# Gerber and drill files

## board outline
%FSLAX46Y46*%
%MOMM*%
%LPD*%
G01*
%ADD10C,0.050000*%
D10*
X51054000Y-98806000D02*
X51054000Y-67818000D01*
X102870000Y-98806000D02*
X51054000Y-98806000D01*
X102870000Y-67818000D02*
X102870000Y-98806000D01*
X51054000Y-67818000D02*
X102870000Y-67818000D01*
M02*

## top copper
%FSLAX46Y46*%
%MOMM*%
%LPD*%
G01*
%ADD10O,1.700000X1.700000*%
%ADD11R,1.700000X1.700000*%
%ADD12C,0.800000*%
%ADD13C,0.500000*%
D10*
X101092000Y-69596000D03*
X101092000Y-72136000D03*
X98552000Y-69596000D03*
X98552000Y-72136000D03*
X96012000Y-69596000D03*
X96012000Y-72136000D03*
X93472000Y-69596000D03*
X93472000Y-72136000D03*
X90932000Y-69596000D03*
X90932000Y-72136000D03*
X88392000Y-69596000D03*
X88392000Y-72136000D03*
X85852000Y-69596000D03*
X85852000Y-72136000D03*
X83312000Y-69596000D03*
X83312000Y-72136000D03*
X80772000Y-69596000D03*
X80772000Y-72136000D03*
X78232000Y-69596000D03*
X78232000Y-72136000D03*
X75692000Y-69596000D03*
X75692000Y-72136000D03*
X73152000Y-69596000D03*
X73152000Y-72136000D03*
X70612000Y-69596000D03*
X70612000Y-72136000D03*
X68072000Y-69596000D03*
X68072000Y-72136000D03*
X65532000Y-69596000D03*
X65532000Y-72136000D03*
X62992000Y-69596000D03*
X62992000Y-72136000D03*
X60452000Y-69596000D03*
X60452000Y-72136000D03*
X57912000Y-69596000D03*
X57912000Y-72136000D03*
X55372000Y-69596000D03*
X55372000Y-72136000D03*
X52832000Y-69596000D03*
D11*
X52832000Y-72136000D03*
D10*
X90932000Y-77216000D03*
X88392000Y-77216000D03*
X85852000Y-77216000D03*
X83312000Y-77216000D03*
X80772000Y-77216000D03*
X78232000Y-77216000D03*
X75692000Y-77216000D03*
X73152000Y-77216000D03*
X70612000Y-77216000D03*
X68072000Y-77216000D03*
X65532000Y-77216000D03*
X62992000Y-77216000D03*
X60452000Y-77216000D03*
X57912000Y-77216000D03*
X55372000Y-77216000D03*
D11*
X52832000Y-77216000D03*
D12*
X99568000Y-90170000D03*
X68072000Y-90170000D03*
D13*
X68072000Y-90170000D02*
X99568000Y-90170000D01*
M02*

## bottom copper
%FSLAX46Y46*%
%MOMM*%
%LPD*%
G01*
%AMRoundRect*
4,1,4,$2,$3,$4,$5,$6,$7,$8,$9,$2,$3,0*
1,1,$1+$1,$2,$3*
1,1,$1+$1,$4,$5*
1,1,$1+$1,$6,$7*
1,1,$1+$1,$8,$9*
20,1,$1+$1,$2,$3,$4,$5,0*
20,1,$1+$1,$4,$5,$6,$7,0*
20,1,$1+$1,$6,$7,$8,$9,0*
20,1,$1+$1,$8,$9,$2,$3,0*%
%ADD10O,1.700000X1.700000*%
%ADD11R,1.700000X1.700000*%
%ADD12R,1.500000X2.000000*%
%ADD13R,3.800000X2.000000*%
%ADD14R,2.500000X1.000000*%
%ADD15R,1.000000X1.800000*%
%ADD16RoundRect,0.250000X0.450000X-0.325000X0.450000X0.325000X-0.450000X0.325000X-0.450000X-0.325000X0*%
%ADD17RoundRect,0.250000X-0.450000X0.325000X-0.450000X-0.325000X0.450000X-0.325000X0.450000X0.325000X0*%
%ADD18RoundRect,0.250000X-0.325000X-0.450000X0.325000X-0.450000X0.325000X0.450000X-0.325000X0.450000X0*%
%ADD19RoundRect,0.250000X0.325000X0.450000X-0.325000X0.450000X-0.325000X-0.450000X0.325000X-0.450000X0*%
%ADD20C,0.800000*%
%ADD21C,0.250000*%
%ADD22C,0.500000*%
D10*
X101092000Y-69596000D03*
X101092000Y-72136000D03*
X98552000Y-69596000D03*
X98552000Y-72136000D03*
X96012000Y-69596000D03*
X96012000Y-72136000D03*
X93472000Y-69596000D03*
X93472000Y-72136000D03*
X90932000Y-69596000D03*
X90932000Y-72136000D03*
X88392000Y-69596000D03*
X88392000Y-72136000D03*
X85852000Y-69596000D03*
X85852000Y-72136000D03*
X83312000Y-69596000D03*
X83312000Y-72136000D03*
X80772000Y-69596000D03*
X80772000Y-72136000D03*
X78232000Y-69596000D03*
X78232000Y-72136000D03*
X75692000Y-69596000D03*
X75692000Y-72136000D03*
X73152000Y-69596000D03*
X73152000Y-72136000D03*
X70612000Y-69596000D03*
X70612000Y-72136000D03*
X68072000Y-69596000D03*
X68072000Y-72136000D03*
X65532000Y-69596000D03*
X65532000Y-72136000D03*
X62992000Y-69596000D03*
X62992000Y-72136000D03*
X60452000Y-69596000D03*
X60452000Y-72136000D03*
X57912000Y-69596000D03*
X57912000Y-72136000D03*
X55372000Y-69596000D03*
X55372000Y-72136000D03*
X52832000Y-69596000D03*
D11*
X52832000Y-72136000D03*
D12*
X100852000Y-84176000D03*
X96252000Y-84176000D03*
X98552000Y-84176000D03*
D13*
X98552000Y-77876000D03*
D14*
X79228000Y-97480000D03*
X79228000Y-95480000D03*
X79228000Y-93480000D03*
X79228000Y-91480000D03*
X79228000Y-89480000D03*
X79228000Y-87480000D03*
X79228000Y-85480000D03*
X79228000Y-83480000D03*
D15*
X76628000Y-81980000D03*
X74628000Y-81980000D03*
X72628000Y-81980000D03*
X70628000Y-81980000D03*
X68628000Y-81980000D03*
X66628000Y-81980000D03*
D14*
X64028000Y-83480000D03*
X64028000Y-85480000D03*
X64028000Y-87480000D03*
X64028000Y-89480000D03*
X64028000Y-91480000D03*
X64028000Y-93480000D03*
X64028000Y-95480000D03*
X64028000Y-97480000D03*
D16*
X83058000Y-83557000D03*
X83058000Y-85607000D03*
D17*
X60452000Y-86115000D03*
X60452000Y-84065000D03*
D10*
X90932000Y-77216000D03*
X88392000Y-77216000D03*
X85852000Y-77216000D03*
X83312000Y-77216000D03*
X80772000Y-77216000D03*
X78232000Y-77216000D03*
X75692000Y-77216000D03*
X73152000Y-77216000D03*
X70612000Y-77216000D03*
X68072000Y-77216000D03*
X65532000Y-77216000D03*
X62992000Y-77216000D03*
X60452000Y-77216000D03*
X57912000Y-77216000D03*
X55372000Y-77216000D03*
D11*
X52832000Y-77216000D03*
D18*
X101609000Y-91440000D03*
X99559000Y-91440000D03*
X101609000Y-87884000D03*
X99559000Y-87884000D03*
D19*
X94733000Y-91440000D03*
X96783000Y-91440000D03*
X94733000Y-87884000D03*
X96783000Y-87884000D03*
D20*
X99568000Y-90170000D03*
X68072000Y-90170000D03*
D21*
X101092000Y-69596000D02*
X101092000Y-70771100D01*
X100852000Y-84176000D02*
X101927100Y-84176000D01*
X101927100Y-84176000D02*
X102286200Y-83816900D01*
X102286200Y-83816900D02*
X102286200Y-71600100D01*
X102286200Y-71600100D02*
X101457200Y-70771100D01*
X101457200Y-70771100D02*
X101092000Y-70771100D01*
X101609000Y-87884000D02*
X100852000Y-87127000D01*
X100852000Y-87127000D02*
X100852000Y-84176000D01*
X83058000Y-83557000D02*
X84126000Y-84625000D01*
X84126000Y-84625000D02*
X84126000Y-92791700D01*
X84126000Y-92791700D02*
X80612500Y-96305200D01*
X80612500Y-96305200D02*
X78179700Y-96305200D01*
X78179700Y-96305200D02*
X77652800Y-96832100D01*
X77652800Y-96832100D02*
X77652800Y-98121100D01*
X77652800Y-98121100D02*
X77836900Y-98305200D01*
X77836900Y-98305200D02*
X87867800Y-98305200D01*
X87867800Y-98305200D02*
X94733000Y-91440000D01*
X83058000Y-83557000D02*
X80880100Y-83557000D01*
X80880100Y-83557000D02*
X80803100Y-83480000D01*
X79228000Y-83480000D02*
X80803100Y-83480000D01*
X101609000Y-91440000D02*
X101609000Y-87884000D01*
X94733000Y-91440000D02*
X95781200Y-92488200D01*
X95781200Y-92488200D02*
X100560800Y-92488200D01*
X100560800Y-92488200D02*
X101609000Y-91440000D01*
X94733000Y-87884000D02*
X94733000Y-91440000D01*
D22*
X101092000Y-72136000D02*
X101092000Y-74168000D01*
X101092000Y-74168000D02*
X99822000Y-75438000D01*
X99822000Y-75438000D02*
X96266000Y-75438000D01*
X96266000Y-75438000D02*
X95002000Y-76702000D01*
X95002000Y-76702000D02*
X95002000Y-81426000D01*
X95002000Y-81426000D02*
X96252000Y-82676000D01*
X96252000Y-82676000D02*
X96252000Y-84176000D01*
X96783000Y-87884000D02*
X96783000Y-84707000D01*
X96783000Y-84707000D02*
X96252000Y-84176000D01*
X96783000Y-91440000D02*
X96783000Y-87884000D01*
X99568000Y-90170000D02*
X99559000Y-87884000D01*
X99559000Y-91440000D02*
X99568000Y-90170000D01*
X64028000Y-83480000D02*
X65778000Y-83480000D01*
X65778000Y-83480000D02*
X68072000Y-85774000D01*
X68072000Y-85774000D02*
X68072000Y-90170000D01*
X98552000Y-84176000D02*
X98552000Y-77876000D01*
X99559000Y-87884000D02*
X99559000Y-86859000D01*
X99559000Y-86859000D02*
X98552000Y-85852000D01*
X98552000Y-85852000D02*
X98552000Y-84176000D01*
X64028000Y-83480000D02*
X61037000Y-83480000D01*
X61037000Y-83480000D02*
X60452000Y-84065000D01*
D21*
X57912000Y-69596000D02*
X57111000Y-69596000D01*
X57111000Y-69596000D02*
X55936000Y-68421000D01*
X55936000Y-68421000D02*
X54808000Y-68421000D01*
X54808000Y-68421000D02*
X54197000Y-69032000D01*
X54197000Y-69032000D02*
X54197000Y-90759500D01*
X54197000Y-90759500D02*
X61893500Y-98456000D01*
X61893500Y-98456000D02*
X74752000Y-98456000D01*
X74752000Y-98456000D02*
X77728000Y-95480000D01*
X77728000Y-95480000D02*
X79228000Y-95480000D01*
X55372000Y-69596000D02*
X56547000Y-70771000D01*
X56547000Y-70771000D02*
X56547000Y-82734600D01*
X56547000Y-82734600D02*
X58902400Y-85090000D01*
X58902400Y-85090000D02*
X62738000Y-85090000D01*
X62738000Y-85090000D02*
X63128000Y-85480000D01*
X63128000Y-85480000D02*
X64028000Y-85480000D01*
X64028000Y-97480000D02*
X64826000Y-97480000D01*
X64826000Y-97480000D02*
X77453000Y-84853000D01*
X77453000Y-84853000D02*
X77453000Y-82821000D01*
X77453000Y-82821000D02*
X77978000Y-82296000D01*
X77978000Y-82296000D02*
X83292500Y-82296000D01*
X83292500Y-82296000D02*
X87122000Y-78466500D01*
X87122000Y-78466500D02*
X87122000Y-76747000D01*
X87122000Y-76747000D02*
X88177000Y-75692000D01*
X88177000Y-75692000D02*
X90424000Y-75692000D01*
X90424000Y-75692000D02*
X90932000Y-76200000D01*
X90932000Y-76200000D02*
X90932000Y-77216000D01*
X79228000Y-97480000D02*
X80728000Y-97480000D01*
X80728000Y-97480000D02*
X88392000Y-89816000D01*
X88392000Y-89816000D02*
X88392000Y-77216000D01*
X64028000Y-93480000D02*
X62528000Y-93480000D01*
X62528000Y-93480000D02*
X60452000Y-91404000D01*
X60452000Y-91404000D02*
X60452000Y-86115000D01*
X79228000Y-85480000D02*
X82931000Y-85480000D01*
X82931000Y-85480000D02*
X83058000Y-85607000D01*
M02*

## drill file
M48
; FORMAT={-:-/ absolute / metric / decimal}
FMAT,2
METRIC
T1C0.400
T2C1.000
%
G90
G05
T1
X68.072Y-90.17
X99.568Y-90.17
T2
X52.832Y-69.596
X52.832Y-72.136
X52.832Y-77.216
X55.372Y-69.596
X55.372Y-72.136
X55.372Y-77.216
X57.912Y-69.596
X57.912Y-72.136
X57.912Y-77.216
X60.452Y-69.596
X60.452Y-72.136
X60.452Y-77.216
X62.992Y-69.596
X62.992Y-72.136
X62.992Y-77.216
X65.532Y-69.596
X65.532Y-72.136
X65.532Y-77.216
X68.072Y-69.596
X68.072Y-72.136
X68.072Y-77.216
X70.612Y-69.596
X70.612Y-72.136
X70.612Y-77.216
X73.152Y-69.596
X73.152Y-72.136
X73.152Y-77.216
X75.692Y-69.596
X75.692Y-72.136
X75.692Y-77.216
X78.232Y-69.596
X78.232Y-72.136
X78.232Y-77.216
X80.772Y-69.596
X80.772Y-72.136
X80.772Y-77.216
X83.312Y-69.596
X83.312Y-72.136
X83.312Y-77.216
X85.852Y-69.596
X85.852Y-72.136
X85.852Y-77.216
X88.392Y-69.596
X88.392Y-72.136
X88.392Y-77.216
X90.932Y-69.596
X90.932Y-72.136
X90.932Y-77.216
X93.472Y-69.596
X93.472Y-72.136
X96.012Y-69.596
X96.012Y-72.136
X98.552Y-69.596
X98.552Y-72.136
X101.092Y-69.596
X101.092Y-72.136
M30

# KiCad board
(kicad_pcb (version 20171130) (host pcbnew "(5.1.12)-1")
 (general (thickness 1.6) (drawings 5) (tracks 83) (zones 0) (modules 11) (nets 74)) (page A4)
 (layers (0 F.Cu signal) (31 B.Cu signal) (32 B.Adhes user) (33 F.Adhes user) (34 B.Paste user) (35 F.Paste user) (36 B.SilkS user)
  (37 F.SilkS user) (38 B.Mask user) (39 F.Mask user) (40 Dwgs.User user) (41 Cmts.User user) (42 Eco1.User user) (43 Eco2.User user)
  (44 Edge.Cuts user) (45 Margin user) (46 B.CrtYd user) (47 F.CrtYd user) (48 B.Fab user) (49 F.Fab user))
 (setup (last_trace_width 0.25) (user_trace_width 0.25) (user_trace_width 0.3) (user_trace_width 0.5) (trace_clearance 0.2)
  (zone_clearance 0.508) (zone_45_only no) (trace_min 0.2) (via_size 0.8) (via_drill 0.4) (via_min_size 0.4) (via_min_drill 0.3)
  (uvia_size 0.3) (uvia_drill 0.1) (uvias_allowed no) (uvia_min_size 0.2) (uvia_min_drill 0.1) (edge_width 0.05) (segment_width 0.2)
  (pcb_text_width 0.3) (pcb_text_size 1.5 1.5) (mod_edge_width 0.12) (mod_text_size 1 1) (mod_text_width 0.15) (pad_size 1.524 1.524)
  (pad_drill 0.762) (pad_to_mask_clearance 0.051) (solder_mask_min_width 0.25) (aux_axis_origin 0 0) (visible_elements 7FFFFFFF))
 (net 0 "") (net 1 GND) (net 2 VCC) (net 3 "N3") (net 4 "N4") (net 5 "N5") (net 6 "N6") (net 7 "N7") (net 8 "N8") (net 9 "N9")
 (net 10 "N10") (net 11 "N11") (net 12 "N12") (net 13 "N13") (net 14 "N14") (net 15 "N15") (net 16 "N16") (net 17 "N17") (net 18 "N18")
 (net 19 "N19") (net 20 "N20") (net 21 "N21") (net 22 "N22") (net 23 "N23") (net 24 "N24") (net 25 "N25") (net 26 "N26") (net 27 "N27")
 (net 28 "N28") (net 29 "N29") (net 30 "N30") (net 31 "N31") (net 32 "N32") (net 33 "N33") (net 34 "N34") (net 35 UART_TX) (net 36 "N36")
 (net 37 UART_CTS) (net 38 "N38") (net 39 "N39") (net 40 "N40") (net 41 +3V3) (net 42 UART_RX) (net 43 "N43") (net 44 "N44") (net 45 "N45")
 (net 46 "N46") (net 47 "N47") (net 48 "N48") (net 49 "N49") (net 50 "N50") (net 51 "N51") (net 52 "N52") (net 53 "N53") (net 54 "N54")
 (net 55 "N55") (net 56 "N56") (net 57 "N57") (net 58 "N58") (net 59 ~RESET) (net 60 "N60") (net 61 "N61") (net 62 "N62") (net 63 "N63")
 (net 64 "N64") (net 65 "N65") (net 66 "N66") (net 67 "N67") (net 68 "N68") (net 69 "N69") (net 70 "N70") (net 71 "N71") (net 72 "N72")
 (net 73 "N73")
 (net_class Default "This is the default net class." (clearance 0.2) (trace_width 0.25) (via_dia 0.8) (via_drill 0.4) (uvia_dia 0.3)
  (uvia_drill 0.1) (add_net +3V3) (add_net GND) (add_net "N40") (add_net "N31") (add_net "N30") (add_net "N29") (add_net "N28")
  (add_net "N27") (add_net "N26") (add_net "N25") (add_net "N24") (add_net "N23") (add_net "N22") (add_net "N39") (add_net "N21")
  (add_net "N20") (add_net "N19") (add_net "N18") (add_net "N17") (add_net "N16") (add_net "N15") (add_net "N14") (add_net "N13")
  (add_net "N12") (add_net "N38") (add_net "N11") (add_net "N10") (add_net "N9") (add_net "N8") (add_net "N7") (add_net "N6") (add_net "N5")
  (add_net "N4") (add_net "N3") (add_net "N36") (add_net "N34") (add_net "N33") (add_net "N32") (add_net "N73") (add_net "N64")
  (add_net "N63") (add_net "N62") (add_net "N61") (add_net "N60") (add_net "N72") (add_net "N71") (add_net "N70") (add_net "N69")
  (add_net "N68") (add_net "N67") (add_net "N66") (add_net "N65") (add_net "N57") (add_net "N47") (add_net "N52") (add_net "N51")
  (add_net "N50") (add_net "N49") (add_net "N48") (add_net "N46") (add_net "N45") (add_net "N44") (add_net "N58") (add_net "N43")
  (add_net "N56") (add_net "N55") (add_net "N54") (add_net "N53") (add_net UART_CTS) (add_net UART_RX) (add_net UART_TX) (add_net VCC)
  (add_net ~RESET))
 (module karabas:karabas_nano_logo (layer F.Cu) (at 83.566 92.456)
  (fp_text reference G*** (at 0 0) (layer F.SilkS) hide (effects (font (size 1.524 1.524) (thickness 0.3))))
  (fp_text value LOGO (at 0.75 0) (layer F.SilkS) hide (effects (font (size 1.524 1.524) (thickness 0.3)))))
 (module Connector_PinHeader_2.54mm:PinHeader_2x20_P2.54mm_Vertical (layer F.Cu) (at 52.832 72.136 90)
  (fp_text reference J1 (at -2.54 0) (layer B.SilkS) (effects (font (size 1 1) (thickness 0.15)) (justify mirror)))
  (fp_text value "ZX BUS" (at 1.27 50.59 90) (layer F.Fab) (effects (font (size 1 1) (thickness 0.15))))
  (pad 40 thru_hole oval (at 2.54 48.26 90) (size 1.7 1.7) (drill 1) (layers *.Cu *.Mask) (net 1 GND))
  (pad 39 thru_hole oval (at 0 48.26 90) (size 1.7 1.7) (drill 1) (layers *.Cu *.Mask) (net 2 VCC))
  (pad 38 thru_hole oval (at 2.54 45.72 90) (size 1.7 1.7) (drill 1) (layers *.Cu *.Mask) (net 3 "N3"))
  (pad 37 thru_hole oval (at 0 45.72 90) (size 1.7 1.7) (drill 1) (layers *.Cu *.Mask) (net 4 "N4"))
  (pad 36 thru_hole oval (at 2.54 43.18 90) (size 1.7 1.7) (drill 1) (layers *.Cu *.Mask) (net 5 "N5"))
  (pad 35 thru_hole oval (at 0 43.18 90) (size 1.7 1.7) (drill 1) (layers *.Cu *.Mask) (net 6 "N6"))
  (pad 34 thru_hole oval (at 2.54 40.64 90) (size 1.7 1.7) (drill 1) (layers *.Cu *.Mask) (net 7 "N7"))
  (pad 33 thru_hole oval (at 0 40.64 90) (size 1.7 1.7) (drill 1) (layers *.Cu *.Mask) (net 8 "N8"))
  (pad 32 thru_hole oval (at 2.54 38.1 90) (size 1.7 1.7) (drill 1) (layers *.Cu *.Mask) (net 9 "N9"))
  (pad 31 thru_hole oval (at 0 38.1 90) (size 1.7 1.7) (drill 1) (layers *.Cu *.Mask) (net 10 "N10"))
  (pad 30 thru_hole oval (at 2.54 35.56 90) (size 1.7 1.7) (drill 1) (layers *.Cu *.Mask) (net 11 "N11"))
  (pad 29 thru_hole oval (at 0 35.56 90) (size 1.7 1.7) (drill 1) (layers *.Cu *.Mask) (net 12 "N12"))
  (pad 28 thru_hole oval (at 2.54 33.02 90) (size 1.7 1.7) (drill 1) (layers *.Cu *.Mask) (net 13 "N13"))
  (pad 27 thru_hole oval (at 0 33.02 90) (size 1.7 1.7) (drill 1) (layers *.Cu *.Mask) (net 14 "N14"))
  (pad 26 thru_hole oval (at 2.54 30.48 90) (size 1.7 1.7) (drill 1) (layers *.Cu *.Mask) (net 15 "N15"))
  (pad 25 thru_hole oval (at 0 30.48 90) (size 1.7 1.7) (drill 1) (layers *.Cu *.Mask) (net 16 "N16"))
  (pad 24 thru_hole oval (at 2.54 27.94 90) (size 1.7 1.7) (drill 1) (layers *.Cu *.Mask) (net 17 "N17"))
  (pad 23 thru_hole oval (at 0 27.94 90) (size 1.7 1.7) (drill 1) (layers *.Cu *.Mask) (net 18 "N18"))
  (pad 22 thru_hole oval (at 2.54 25.4 90) (size 1.7 1.7) (drill 1) (layers *.Cu *.Mask) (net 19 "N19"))
  (pad 21 thru_hole oval (at 0 25.4 90) (size 1.7 1.7) (drill 1) (layers *.Cu *.Mask) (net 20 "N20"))
  (pad 20 thru_hole oval (at 2.54 22.86 90) (size 1.7 1.7) (drill 1) (layers *.Cu *.Mask) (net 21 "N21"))
  (pad 19 thru_hole oval (at 0 22.86 90) (size 1.7 1.7) (drill 1) (layers *.Cu *.Mask) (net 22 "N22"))
  (pad 18 thru_hole oval (at 2.54 20.32 90) (size 1.7 1.7) (drill 1) (layers *.Cu *.Mask) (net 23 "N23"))
  (pad 17 thru_hole oval (at 0 20.32 90) (size 1.7 1.7) (drill 1) (layers *.Cu *.Mask) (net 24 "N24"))
  (pad 16 thru_hole oval (at 2.54 17.78 90) (size 1.7 1.7) (drill 1) (layers *.Cu *.Mask) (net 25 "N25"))
  (pad 15 thru_hole oval (at 0 17.78 90) (size 1.7 1.7) (drill 1) (layers *.Cu *.Mask) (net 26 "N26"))
  (pad 14 thru_hole oval (at 2.54 15.24 90) (size 1.7 1.7) (drill 1) (layers *.Cu *.Mask) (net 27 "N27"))
  (pad 13 thru_hole oval (at 0 15.24 90) (size 1.7 1.7) (drill 1) (layers *.Cu *.Mask) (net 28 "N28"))
  (pad 12 thru_hole oval (at 2.54 12.7 90) (size 1.7 1.7) (drill 1) (layers *.Cu *.Mask) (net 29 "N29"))
  (pad 11 thru_hole oval (at 0 12.7 90) (size 1.7 1.7) (drill 1) (layers *.Cu *.Mask) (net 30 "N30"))
  (pad 10 thru_hole oval (at 2.54 10.16 90) (size 1.7 1.7) (drill 1) (layers *.Cu *.Mask) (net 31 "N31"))
  (pad 9 thru_hole oval (at 0 10.16 90) (size 1.7 1.7) (drill 1) (layers *.Cu *.Mask) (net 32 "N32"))
  (pad 8 thru_hole oval (at 2.54 7.62 90) (size 1.7 1.7) (drill 1) (layers *.Cu *.Mask) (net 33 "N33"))
  (pad 7 thru_hole oval (at 0 7.62 90) (size 1.7 1.7) (drill 1) (layers *.Cu *.Mask) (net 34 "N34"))
  (pad 6 thru_hole oval (at 2.54 5.08 90) (size 1.7 1.7) (drill 1) (layers *.Cu *.Mask) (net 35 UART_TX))
  (pad 5 thru_hole oval (at 0 5.08 90) (size 1.7 1.7) (drill 1) (layers *.Cu *.Mask) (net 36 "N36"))
  (pad 4 thru_hole oval (at 2.54 2.54 90) (size 1.7 1.7) (drill 1) (layers *.Cu *.Mask) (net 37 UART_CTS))
  (pad 3 thru_hole oval (at 0 2.54 90) (size 1.7 1.7) (drill 1) (layers *.Cu *.Mask) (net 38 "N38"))
  (pad 2 thru_hole oval (at 2.54 0 90) (size 1.7 1.7) (drill 1) (layers *.Cu *.Mask) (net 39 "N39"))
  (pad 1 thru_hole rect (at 0 0 90) (size 1.7 1.7) (drill 1) (layers *.Cu *.Mask) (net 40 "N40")))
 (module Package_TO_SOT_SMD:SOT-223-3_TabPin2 (layer B.Cu) (at 98.552 81.026 90)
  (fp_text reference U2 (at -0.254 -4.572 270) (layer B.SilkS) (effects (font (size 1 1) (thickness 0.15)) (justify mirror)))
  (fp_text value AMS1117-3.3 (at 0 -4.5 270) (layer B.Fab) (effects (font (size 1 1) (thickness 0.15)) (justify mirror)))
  (pad 1 smd rect (at -3.15 2.3 90) (size 2 1.5) (layers B.Cu B.Paste B.Mask) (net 1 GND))
  (pad 3 smd rect (at -3.15 -2.3 90) (size 2 1.5) (layers B.Cu B.Paste B.Mask) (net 2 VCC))
  (pad 2 smd rect (at -3.15 0 90) (size 2 1.5) (layers B.Cu B.Paste B.Mask) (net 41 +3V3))
  (pad 2 smd rect (at 3.15 0 90) (size 2 3.8) (layers B.Cu B.Paste B.Mask) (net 41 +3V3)))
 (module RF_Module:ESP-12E (layer B.Cu) (at 71.628 93.98)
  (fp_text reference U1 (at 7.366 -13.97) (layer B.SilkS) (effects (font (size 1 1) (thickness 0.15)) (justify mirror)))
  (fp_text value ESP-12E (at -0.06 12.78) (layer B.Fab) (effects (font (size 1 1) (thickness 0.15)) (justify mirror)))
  (pad 22 smd rect (at 7.6 3.5) (size 2.5 1) (layers B.Cu B.Paste B.Mask) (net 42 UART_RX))
  (pad 21 smd rect (at 7.6 1.5) (size 2.5 1) (layers B.Cu B.Paste B.Mask) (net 35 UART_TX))
  (pad 20 smd rect (at 7.6 -0.5) (size 2.5 1) (layers B.Cu B.Paste B.Mask) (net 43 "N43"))
  (pad 19 smd rect (at 7.6 -2.5) (size 2.5 1) (layers B.Cu B.Paste B.Mask) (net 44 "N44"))
  (pad 18 smd rect (at 7.6 -4.5) (size 2.5 1) (layers B.Cu B.Paste B.Mask) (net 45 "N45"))
  (pad 17 smd rect (at 7.6 -6.5) (size 2.5 1) (layers B.Cu B.Paste B.Mask) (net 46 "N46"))
  (pad 16 smd rect (at 7.6 -8.5) (size 2.5 1) (layers B.Cu B.Paste B.Mask) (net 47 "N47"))
  (pad 15 smd rect (at 7.6 -10.5) (size 2.5 1) (layers B.Cu B.Paste B.Mask) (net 1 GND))
  (pad 14 smd rect (at 5 -12) (size 1 1.8) (layers B.Cu B.Paste B.Mask) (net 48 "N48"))
  (pad 13 smd rect (at 3 -12) (size 1 1.8) (layers B.Cu B.Paste B.Mask) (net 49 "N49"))
  (pad 12 smd rect (at 1 -12) (size 1 1.8) (layers B.Cu B.Paste B.Mask) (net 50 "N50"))
  (pad 11 smd rect (at -1 -12) (size 1 1.8) (layers B.Cu B.Paste B.Mask) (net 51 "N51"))
  (pad 10 smd rect (at -3 -12) (size 1 1.8) (layers B.Cu B.Paste B.Mask) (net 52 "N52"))
  (pad 9 smd rect (at -5 -12) (size 1 1.8) (layers B.Cu B.Paste B.Mask) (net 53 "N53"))
  (pad 8 smd rect (at -7.6 -10.5) (size 2.5 1) (layers B.Cu B.Paste B.Mask) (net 41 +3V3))
  (pad 7 smd rect (at -7.6 -8.5) (size 2.5 1) (layers B.Cu B.Paste B.Mask) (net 37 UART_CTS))
  (pad 6 smd rect (at -7.6 -6.5) (size 2.5 1) (layers B.Cu B.Paste B.Mask) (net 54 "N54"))
  (pad 5 smd rect (at -7.6 -4.5) (size 2.5 1) (layers B.Cu B.Paste B.Mask) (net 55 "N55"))
  (pad 4 smd rect (at -7.6 -2.5) (size 2.5 1) (layers B.Cu B.Paste B.Mask) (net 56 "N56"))
  (pad 3 smd rect (at -7.6 -0.5) (size 2.5 1) (layers B.Cu B.Paste B.Mask) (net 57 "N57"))
  (pad 2 smd rect (at -7.6 1.5) (size 2.5 1) (layers B.Cu B.Paste B.Mask) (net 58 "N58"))
  (pad 1 smd rect (at -7.6 3.5) (size 2.5 1) (layers B.Cu B.Paste B.Mask) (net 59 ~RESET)))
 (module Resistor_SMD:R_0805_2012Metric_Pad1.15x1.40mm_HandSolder (layer B.Cu) (at 83.058 84.582 90)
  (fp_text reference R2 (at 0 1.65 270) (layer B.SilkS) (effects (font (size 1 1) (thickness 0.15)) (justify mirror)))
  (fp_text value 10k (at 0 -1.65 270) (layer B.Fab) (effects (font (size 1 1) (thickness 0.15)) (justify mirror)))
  (pad 2 smd roundrect (at 1.025 0 90) (size 1.15 1.4) (layers B.Cu B.Paste B.Mask) (roundrect_rratio 0.217391) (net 1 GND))
  (pad 1 smd roundrect (at -1.025 0 90) (size 1.15 1.4) (layers B.Cu B.Paste B.Mask) (roundrect_rratio 0.217391) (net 47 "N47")))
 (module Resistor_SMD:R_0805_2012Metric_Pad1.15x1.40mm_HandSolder (layer B.Cu) (at 60.452 85.09 270)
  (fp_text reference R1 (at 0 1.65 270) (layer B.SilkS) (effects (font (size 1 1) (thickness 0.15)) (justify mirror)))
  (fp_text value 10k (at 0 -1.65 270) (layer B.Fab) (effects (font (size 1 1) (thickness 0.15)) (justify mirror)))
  (pad 2 smd roundrect (at 1.025 0 270) (size 1.15 1.4) (layers B.Cu B.Paste B.Mask) (roundrect_rratio 0.217391) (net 57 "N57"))
  (pad 1 smd roundrect (at -1.025 0 270) (size 1.15 1.4) (layers B.Cu B.Paste B.Mask) (roundrect_rratio 0.217391) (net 41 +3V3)))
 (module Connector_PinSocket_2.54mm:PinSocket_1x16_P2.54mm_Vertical (layer F.Cu) (at 52.832 77.216 90)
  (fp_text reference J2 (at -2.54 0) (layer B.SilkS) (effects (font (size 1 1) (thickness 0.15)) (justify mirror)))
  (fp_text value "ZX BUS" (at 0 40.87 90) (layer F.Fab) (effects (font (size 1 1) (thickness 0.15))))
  (pad 16 thru_hole oval (at 0 38.1 90) (size 1.7 1.7) (drill 1) (layers *.Cu *.Mask) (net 59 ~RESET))
  (pad 15 thru_hole oval (at 0 35.56 90) (size 1.7 1.7) (drill 1) (layers *.Cu *.Mask) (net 42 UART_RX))
  (pad 14 thru_hole oval (at 0 33.02 90) (size 1.7 1.7) (drill 1) (layers *.Cu *.Mask) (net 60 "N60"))
  (pad 13 thru_hole oval (at 0 30.48 90) (size 1.7 1.7) (drill 1) (layers *.Cu *.Mask) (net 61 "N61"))
  (pad 12 thru_hole oval (at 0 27.94 90) (size 1.7 1.7) (drill 1) (layers *.Cu *.Mask) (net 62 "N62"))
  (pad 11 thru_hole oval (at 0 25.4 90) (size 1.7 1.7) (drill 1) (layers *.Cu *.Mask) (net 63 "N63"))
  (pad 10 thru_hole oval (at 0 22.86 90) (size 1.7 1.7) (drill 1) (layers *.Cu *.Mask) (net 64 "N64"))
  (pad 9 thru_hole oval (at 0 20.32 90) (size 1.7 1.7) (drill 1) (layers *.Cu *.Mask) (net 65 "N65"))
  (pad 8 thru_hole oval (at 0 17.78 90) (size 1.7 1.7) (drill 1) (layers *.Cu *.Mask) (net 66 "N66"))
  (pad 7 thru_hole oval (at 0 15.24 90) (size 1.7 1.7) (drill 1) (layers *.Cu *.Mask) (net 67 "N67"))
  (pad 6 thru_hole oval (at 0 12.7 90) (size 1.7 1.7) (drill 1) (layers *.Cu *.Mask) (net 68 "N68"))
  (pad 5 thru_hole oval (at 0 10.16 90) (size 1.7 1.7) (drill 1) (layers *.Cu *.Mask) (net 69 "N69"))
  (pad 4 thru_hole oval (at 0 7.62 90) (size 1.7 1.7) (drill 1) (layers *.Cu *.Mask) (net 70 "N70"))
  (pad 3 thru_hole oval (at 0 5.08 90) (size 1.7 1.7) (drill 1) (layers *.Cu *.Mask) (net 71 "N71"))
  (pad 2 thru_hole oval (at 0 2.54 90) (size 1.7 1.7) (drill 1) (layers *.Cu *.Mask) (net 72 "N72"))
  (pad 1 thru_hole rect (at 0 0 90) (size 1.7 1.7) (drill 1) (layers *.Cu *.Mask) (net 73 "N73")))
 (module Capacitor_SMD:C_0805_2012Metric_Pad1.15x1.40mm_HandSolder (layer B.Cu) (at 100.584 91.44)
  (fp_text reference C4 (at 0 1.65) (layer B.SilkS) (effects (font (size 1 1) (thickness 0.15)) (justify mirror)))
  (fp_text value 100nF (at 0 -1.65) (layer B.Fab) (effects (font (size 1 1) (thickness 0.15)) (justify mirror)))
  (pad 2 smd roundrect (at 1.025 0) (size 1.15 1.4) (layers B.Cu B.Paste B.Mask) (roundrect_rratio 0.217391) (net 1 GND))
  (pad 1 smd roundrect (at -1.025 0) (size 1.15 1.4) (layers B.Cu B.Paste B.Mask) (roundrect_rratio 0.217391) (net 41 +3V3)))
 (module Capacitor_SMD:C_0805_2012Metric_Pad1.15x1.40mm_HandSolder (layer B.Cu) (at 100.584 87.884)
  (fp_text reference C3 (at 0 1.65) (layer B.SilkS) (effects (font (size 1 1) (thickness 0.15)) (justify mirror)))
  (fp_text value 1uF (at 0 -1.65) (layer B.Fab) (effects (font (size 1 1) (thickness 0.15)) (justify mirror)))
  (pad 2 smd roundrect (at 1.025 0) (size 1.15 1.4) (layers B.Cu B.Paste B.Mask) (roundrect_rratio 0.217391) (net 1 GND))
  (pad 1 smd roundrect (at -1.025 0) (size 1.15 1.4) (layers B.Cu B.Paste B.Mask) (roundrect_rratio 0.217391) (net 41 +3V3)))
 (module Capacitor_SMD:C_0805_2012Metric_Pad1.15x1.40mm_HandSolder (layer B.Cu) (at 95.758 91.44 180)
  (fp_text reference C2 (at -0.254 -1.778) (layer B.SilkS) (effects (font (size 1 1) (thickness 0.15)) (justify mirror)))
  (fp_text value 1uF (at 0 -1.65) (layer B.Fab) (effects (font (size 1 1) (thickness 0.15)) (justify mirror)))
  (pad 2 smd roundrect (at 1.025 0 180) (size 1.15 1.4) (layers B.Cu B.Paste B.Mask) (roundrect_rratio 0.217391) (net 1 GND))
  (pad 1 smd roundrect (at -1.025 0 180) (size 1.15 1.4) (layers B.Cu B.Paste B.Mask) (roundrect_rratio 0.217391) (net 2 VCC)))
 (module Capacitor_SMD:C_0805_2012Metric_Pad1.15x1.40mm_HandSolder (layer B.Cu) (at 95.758 87.884 180)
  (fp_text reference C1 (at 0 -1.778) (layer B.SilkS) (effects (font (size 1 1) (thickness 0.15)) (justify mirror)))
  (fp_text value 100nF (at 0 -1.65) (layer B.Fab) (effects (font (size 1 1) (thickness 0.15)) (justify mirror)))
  (pad 2 smd roundrect (at 1.025 0 180) (size 1.15 1.4) (layers B.Cu B.Paste B.Mask) (roundrect_rratio 0.217391) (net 1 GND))
  (pad 1 smd roundrect (at -1.025 0 180) (size 1.15 1.4) (layers B.Cu B.Paste B.Mask) (roundrect_rratio 0.217391) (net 2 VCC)))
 (gr_line (start 51.054 98.806) (end 51.054 67.818) (layer Edge.Cuts) (width 0.05))
 (gr_line (start 102.87 98.806) (end 51.054 98.806) (layer Edge.Cuts) (width 0.05))
 (gr_line (start 102.87 67.818) (end 102.87 98.806) (layer Edge.Cuts) (width 0.05))
 (gr_line (start 51.054 67.818) (end 102.87 67.818) (layer Edge.Cuts) (width 0.05))
 (segment (start 101.092 69.596) (end 101.092 70.7711) (width 0.25) (layer B.Cu) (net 1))
 (segment (start 100.852 84.176) (end 101.9271 84.176) (width 0.25) (layer B.Cu) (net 1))
 (segment (start 101.9271 84.176) (end 102.2862 83.8169) (width 0.25) (layer B.Cu) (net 1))
 (segment (start 102.2862 83.8169) (end 102.2862 71.6001) (width 0.25) (layer B.Cu) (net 1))
 (segment (start 102.2862 71.6001) (end 101.4572 70.7711) (width 0.25) (layer B.Cu) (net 1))
 (segment (start 101.4572 70.7711) (end 101.092 70.7711) (width 0.25) (layer B.Cu) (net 1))
 (segment (start 101.609 87.884) (end 100.852 87.127) (width 0.25) (layer B.Cu) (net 1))
 (segment (start 100.852 87.127) (end 100.852 84.176) (width 0.25) (layer B.Cu) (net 1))
 (segment (start 83.058 83.557) (end 84.126 84.625) (width 0.25) (layer B.Cu) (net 1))
 (segment (start 84.126 84.625) (end 84.126 92.7917) (width 0.25) (layer B.Cu) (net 1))
 (segment (start 84.126 92.7917) (end 80.6125 96.3052) (width 0.25) (layer B.Cu) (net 1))
 (segment (start 80.6125 96.3052) (end 78.1797 96.3052) (width 0.25) (layer B.Cu) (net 1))
 (segment (start 78.1797 96.3052) (end 77.6528 96.8321) (width 0.25) (layer B.Cu) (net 1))
 (segment (start 77.6528 96.8321) (end 77.6528 98.1211) (width 0.25) (layer B.Cu) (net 1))
 (segment (start 77.6528 98.1211) (end 77.8369 98.3052) (width 0.25) (layer B.Cu) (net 1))
 (segment (start 77.8369 98.3052) (end 87.8678 98.3052) (width 0.25) (layer B.Cu) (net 1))
 (segment (start 87.8678 98.3052) (end 94.733 91.44) (width 0.25) (layer B.Cu) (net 1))
 (segment (start 83.058 83.557) (end 80.8801 83.557) (width 0.25) (layer B.Cu) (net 1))
 (segment (start 80.8801 83.557) (end 80.8031 83.48) (width 0.25) (layer B.Cu) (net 1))
 (segment (start 79.228 83.48) (end 80.8031 83.48) (width 0.25) (layer B.Cu) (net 1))
 (segment (start 101.609 91.44) (end 101.609 87.884) (width 0.25) (layer B.Cu) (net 1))
 (segment (start 94.733 91.44) (end 95.7812 92.4882) (width 0.25) (layer B.Cu) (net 1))
 (segment (start 95.7812 92.4882) (end 100.5608 92.4882) (width 0.25) (layer B.Cu) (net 1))
 (segment (start 100.5608 92.4882) (end 101.609 91.44) (width 0.25) (layer B.Cu) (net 1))
 (segment (start 94.733 87.884) (end 94.733 91.44) (width 0.25) (layer B.Cu) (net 1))
 (segment (start 101.092 72.136) (end 101.092 74.168) (width 0.5) (layer B.Cu) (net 2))
 (segment (start 101.092 74.168) (end 99.822 75.438) (width 0.5) (layer B.Cu) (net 2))
 (segment (start 99.822 75.438) (end 96.266 75.438) (width 0.5) (layer B.Cu) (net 2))
 (segment (start 96.266 75.438) (end 95.002 76.702) (width 0.5) (layer B.Cu) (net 2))
 (segment (start 95.002 76.702) (end 95.002 81.426) (width 0.5) (layer B.Cu) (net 2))
 (segment (start 95.002 81.426) (end 96.252 82.676) (width 0.5) (layer B.Cu) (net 2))
 (segment (start 96.252 82.676) (end 96.252 84.176) (width 0.5) (layer B.Cu) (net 2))
 (segment (start 96.783 87.884) (end 96.783 84.707) (width 0.5) (layer B.Cu) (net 2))
 (segment (start 96.783 84.707) (end 96.252 84.176) (width 0.5) (layer B.Cu) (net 2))
 (segment (start 96.783 91.44) (end 96.783 87.884) (width 0.5) (layer B.Cu) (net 2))
 (segment (start 99.568 90.17) (end 99.559 87.884) (width 0.5) (layer B.Cu) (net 41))
 (segment (start 99.559 91.44) (end 99.568 90.17) (width 0.5) (layer B.Cu) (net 41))
 (segment (start 68.072 90.17) (end 99.568 90.17) (width 0.5) (layer F.Cu) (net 41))
 (segment (start 64.028 83.48) (end 65.778 83.48) (width 0.5) (layer B.Cu) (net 41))
 (segment (start 65.778 83.48) (end 68.072 85.774) (width 0.5) (layer B.Cu) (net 41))
 (segment (start 68.072 85.774) (end 68.072 90.17) (width 0.5) (layer B.Cu) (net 41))
 (segment (start 98.552 84.176) (end 98.552 77.876) (width 0.5) (layer B.Cu) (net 41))
 (segment (start 99.559 87.884) (end 99.559 86.859) (width 0.5) (layer B.Cu) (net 41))
 (segment (start 99.559 86.859) (end 98.552 85.852) (width 0.5) (layer B.Cu) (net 41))
 (segment (start 98.552 85.852) (end 98.552 84.176) (width 0.5) (layer B.Cu) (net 41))
 (segment (start 64.028 83.48) (end 61.037 83.48) (width 0.5) (layer B.Cu) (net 41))
 (segment (start 61.037 83.48) (end 60.452 84.065) (width 0.5) (layer B.Cu) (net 41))
 (via (at 99.568 90.17) (size 0.8) (layers F.Cu B.Cu) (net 41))
 (via (at 68.072 90.17) (size 0.8) (layers F.Cu B.Cu) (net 41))
 (segment (start 57.912 69.596) (end 57.111 69.596) (width 0.25) (layer B.Cu) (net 35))
 (segment (start 57.111 69.596) (end 55.936 68.421) (width 0.25) (layer B.Cu) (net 35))
 (segment (start 55.936 68.421) (end 54.808 68.421) (width 0.25) (layer B.Cu) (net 35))
 (segment (start 54.808 68.421) (end 54.197 69.032) (width 0.25) (layer B.Cu) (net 35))
 (segment (start 54.197 69.032) (end 54.197 90.7595) (width 0.25) (layer B.Cu) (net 35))
 (segment (start 54.197 90.7595) (end 61.8935 98.456) (width 0.25) (layer B.Cu) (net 35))
 (segment (start 61.8935 98.456) (end 74.752 98.456) (width 0.25) (layer B.Cu) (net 35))
 (segment (start 74.752 98.456) (end 77.728 95.48) (width 0.25) (layer B.Cu) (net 35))
 (segment (start 77.728 95.48) (end 79.228 95.48) (width 0.25) (layer B.Cu) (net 35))
 (segment (start 55.372 69.596) (end 56.547 70.771) (width 0.25) (layer B.Cu) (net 37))
 (segment (start 56.547 70.771) (end 56.547 82.7346) (width 0.25) (layer B.Cu) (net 37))
 (segment (start 56.547 82.7346) (end 58.9024 85.09) (width 0.25) (layer B.Cu) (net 37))
 (segment (start 58.9024 85.09) (end 62.738 85.09) (width 0.25) (layer B.Cu) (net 37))
 (segment (start 62.738 85.09) (end 63.128 85.48) (width 0.25) (layer B.Cu) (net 37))
 (segment (start 63.128 85.48) (end 64.028 85.48) (width 0.25) (layer B.Cu) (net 37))
 (segment (start 64.028 97.48) (end 64.826 97.48) (width 0.25) (layer B.Cu) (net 59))
 (segment (start 64.826 97.48) (end 77.453 84.853) (width 0.25) (layer B.Cu) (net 59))
 (segment (start 77.453 84.853) (end 77.453 82.821) (width 0.25) (layer B.Cu) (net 59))
 (segment (start 77.453 82.821) (end 77.978 82.296) (width 0.25) (layer B.Cu) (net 59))
 (segment (start 77.978 82.296) (end 83.2925 82.296) (width 0.25) (layer B.Cu) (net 59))
 (segment (start 83.2925 82.296) (end 87.122 78.4665) (width 0.25) (layer B.Cu) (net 59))
 (segment (start 87.122 78.4665) (end 87.122 76.747) (width 0.25) (layer B.Cu) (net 59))
 (segment (start 87.122 76.747) (end 88.177 75.692) (width 0.25) (layer B.Cu) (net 59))
 (segment (start 88.177 75.692) (end 90.424 75.692) (width 0.25) (layer B.Cu) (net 59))
 (segment (start 90.424 75.692) (end 90.932 76.2) (width 0.25) (layer B.Cu) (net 59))
 (segment (start 90.932 76.2) (end 90.932 77.216) (width 0.25) (layer B.Cu) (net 59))
 (segment (start 79.228 97.48) (end 80.728 97.48) (width 0.25) (layer B.Cu) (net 42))
 (segment (start 80.728 97.48) (end 88.392 89.816) (width 0.25) (layer B.Cu) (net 42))
 (segment (start 88.392 89.816) (end 88.392 77.216) (width 0.25) (layer B.Cu) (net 42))
 (segment (start 64.028 93.48) (end 62.528 93.48) (width 0.25) (layer B.Cu) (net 57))
 (segment (start 62.528 93.48) (end 60.452 91.404) (width 0.25) (layer B.Cu) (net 57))
 (segment (start 60.452 91.404) (end 60.452 86.115) (width 0.25) (layer B.Cu) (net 57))
 (segment (start 79.228 85.48) (end 82.931 85.48) (width 0.25) (layer B.Cu) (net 47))
 (segment (start 82.931 85.48) (end 83.058 85.607) (width 0.25) (layer B.Cu) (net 47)))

